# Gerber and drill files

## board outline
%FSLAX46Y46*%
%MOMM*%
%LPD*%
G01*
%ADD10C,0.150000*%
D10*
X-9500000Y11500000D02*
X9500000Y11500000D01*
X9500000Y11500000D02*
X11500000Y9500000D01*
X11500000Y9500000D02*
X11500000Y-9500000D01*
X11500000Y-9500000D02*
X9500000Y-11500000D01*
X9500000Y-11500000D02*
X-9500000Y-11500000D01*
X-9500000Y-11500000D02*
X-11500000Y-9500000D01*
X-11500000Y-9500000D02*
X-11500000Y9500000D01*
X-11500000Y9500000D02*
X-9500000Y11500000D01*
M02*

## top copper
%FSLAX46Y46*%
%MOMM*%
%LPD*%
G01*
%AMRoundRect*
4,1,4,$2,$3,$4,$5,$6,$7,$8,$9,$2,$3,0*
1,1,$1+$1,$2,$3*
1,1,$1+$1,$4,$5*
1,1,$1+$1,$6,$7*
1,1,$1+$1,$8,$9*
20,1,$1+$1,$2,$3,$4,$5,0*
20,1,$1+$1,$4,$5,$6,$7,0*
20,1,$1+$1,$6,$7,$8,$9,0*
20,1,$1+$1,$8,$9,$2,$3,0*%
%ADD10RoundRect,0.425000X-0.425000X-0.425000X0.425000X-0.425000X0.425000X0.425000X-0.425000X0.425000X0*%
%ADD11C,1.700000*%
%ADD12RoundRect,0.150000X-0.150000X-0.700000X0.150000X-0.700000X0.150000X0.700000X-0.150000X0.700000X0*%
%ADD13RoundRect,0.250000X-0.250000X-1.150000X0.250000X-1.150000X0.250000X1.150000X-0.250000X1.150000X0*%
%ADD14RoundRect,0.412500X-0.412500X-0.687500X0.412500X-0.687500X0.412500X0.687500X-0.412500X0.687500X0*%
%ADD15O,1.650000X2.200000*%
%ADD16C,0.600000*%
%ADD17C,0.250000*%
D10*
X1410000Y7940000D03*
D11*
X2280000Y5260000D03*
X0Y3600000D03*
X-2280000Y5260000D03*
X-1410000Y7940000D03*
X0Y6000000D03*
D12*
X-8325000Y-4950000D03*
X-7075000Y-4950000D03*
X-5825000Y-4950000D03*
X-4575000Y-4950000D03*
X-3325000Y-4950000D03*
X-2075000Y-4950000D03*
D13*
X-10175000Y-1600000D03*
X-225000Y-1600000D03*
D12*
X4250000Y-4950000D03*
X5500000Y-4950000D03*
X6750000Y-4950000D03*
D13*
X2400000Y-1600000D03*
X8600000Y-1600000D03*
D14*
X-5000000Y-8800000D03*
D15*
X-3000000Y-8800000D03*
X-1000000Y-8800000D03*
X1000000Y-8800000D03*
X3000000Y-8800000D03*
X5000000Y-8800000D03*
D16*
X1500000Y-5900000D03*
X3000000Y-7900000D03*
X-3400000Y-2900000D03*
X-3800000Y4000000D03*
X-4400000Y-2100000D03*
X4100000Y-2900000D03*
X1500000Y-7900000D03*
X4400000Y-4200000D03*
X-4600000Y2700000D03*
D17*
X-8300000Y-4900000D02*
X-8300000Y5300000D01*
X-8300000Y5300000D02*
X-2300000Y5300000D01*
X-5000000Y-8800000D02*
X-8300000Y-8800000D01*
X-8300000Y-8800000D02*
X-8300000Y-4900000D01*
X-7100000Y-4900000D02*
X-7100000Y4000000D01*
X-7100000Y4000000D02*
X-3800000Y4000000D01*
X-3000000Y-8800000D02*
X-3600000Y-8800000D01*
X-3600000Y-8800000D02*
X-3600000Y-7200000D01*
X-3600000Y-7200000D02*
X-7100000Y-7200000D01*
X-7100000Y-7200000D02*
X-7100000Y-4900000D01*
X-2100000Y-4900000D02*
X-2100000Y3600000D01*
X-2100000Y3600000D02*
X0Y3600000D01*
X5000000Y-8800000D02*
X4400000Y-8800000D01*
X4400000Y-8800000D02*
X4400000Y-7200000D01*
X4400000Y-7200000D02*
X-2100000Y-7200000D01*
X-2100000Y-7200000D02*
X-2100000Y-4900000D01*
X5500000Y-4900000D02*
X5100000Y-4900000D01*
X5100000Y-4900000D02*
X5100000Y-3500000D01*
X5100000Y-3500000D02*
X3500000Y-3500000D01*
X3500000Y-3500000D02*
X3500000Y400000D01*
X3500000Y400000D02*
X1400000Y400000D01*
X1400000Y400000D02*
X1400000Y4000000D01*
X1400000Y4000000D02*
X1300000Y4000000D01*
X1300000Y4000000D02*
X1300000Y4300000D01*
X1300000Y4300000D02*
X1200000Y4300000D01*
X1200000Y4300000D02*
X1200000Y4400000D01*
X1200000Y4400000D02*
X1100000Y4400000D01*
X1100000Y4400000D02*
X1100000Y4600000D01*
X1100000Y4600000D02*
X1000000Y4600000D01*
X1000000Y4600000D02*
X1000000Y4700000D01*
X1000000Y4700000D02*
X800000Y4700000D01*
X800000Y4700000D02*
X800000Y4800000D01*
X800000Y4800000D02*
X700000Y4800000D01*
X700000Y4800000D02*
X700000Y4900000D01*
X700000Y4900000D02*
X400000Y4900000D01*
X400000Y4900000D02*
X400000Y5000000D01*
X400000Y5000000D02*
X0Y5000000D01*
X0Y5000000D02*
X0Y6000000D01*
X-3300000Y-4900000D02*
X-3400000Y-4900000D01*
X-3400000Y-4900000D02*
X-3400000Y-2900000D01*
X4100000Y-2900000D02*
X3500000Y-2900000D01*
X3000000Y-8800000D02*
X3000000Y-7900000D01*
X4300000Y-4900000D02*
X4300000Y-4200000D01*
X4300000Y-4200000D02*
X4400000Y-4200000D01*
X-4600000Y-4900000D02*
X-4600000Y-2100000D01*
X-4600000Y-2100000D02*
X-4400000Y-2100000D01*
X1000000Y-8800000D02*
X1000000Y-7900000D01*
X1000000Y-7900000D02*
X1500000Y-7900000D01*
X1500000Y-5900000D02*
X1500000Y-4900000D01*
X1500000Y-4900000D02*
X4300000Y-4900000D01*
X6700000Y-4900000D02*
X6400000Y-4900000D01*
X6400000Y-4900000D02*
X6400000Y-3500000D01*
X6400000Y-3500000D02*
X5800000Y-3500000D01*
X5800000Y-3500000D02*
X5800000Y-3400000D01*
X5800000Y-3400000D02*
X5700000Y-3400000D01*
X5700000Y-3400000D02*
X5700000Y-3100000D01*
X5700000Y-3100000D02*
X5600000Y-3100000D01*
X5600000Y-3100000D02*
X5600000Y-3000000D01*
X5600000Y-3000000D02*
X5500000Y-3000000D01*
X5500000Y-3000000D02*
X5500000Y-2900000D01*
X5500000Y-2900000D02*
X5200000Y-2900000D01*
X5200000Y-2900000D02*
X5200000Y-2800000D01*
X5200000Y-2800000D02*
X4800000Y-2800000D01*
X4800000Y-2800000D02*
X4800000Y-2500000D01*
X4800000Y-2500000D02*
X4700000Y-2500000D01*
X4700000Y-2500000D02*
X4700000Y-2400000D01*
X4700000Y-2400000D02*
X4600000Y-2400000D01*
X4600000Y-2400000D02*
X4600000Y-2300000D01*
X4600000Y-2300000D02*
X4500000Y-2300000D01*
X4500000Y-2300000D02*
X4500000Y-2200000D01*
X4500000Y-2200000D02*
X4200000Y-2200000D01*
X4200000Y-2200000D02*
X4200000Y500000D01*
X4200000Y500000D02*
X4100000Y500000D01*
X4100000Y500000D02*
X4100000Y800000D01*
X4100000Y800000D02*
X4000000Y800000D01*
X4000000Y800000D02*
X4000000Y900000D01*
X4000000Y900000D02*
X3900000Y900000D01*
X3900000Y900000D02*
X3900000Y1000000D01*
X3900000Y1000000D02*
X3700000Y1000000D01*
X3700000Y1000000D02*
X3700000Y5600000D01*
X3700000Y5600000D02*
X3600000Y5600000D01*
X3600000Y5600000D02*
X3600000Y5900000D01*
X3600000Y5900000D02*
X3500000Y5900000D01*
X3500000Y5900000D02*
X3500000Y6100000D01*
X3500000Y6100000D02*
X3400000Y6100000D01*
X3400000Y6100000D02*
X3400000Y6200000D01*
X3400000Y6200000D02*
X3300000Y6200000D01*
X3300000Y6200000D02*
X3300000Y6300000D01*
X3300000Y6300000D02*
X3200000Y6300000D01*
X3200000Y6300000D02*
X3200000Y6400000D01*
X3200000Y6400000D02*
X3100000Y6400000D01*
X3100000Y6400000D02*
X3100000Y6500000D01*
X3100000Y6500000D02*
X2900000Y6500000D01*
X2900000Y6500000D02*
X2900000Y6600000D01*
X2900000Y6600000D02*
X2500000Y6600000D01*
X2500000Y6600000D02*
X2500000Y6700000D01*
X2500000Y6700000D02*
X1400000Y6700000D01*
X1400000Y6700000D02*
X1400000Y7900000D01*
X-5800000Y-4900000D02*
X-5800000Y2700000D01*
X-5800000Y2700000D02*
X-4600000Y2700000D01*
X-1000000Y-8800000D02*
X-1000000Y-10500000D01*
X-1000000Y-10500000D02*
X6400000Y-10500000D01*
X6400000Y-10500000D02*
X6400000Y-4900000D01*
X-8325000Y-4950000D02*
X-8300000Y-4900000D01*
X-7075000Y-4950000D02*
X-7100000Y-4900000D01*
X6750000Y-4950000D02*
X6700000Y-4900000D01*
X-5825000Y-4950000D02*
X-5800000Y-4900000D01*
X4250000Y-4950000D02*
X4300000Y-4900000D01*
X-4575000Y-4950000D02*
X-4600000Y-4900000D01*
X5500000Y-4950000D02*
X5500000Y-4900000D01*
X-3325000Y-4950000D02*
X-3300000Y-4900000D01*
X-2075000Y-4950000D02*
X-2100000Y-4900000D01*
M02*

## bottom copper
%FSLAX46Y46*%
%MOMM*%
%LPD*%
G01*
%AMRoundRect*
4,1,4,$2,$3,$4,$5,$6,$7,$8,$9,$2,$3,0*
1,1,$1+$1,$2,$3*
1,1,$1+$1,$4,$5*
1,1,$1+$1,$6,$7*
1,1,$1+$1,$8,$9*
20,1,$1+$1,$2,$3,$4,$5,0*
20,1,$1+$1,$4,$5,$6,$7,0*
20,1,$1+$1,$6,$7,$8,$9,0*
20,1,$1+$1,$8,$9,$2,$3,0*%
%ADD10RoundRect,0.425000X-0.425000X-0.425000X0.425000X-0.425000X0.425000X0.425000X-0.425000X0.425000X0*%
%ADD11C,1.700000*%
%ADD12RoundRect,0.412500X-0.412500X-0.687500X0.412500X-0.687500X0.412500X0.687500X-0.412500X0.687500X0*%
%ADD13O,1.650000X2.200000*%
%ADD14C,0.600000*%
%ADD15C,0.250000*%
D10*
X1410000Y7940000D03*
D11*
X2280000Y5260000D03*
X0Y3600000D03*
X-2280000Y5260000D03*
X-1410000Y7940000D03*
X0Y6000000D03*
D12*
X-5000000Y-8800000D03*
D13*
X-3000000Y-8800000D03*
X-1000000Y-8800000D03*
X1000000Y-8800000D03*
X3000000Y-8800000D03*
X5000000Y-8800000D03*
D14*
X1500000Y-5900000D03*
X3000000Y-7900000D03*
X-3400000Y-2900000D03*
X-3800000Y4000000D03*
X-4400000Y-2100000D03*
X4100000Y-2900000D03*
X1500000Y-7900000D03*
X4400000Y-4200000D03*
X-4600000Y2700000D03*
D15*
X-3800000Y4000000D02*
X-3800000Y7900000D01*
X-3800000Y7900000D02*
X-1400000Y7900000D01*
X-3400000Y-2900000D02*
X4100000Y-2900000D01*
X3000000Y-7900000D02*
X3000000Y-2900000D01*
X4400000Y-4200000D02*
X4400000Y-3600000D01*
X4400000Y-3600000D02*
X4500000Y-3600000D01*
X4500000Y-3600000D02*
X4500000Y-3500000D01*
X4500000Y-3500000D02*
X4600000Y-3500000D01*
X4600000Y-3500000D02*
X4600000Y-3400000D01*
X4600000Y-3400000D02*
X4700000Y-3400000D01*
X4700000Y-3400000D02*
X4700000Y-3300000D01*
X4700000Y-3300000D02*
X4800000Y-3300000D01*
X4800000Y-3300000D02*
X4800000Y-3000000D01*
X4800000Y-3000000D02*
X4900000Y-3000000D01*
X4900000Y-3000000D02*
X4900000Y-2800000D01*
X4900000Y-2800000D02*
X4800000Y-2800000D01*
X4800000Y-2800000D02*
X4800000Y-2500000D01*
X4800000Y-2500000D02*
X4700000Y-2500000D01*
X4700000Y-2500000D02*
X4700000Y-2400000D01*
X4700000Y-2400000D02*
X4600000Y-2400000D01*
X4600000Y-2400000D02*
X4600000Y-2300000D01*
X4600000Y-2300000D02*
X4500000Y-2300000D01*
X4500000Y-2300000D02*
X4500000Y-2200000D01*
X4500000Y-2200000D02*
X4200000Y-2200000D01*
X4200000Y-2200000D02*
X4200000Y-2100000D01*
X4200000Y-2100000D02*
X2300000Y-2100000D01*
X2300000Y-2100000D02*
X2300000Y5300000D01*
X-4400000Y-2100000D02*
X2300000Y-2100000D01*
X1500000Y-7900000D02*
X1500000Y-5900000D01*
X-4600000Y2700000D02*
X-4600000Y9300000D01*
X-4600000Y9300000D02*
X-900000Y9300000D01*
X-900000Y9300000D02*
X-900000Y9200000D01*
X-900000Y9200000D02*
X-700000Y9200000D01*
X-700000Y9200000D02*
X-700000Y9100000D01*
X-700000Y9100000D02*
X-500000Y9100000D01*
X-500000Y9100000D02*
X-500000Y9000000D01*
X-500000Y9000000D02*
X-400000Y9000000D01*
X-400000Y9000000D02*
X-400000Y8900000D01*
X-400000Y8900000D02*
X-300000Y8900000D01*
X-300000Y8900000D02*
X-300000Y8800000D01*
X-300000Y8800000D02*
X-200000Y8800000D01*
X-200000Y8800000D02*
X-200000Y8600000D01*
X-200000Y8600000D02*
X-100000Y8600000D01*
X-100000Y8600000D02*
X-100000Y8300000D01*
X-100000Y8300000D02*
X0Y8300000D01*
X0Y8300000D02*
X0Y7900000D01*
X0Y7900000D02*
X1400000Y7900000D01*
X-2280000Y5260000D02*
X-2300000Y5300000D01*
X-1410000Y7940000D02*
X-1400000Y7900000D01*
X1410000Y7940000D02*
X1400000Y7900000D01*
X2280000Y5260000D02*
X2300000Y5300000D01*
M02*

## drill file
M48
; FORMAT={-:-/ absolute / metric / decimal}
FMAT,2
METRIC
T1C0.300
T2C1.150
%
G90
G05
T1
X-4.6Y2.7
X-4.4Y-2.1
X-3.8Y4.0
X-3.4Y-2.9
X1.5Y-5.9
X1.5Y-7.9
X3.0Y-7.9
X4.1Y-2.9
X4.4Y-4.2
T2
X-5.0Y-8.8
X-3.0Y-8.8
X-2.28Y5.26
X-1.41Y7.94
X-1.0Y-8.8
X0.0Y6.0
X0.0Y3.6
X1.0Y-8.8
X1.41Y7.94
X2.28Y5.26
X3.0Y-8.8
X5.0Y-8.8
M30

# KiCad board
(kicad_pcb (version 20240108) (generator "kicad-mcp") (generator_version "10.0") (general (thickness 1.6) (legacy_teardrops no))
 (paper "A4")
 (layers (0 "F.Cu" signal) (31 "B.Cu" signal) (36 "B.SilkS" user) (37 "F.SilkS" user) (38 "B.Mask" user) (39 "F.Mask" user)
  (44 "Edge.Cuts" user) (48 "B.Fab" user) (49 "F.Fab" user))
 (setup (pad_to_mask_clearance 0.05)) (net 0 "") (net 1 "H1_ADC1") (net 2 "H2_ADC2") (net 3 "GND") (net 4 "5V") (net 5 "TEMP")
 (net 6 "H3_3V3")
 (gr_line (start -9.5 -11.5) (end 9.5 -11.5) (stroke (width 0.15) (type solid)) (layer "Edge.Cuts"))
 (gr_line (start 9.5 -11.5) (end 11.5 -9.5) (stroke (width 0.15) (type solid)) (layer "Edge.Cuts"))
 (gr_line (start 11.5 -9.5) (end 11.5 9.5) (stroke (width 0.15) (type solid)) (layer "Edge.Cuts"))
 (gr_line (start 11.5 9.5) (end 9.5 11.5) (stroke (width 0.15) (type solid)) (layer "Edge.Cuts"))
 (gr_line (start 9.5 11.5) (end -9.5 11.5) (stroke (width 0.15) (type solid)) (layer "Edge.Cuts"))
 (gr_line (start -9.5 11.5) (end -11.5 9.5) (stroke (width 0.15) (type solid)) (layer "Edge.Cuts"))
 (gr_line (start -11.5 9.5) (end -11.5 -9.5) (stroke (width 0.15) (type solid)) (layer "Edge.Cuts"))
 (gr_line (start -11.5 -9.5) (end -9.5 -11.5) (stroke (width 0.15) (type solid)) (layer "Edge.Cuts"))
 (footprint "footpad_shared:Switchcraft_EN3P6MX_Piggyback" (layer "F.Cu") (at 0 -6.0 0)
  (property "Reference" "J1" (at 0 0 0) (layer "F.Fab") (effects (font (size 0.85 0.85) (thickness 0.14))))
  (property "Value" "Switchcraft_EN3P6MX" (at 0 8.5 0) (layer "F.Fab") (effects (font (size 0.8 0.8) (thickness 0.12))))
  (pad "1" thru_hole roundrect (at 1.41 -1.94) (size 1.7 1.7) (drill 1.15) (layers "*.Cu" "*.Mask") (roundrect_rratio 0.25)
   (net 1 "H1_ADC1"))
  (pad "2" thru_hole circle (at 2.28 0.74) (size 1.7 1.7) (drill 1.15) (layers "*.Cu" "*.Mask") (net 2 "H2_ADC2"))
  (pad "3" thru_hole circle (at 0 2.4) (size 1.7 1.7) (drill 1.15) (layers "*.Cu" "*.Mask") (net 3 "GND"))
  (pad "4" thru_hole circle (at -2.28 0.74) (size 1.7 1.7) (drill 1.15) (layers "*.Cu" "*.Mask") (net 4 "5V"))
  (pad "5" thru_hole circle (at -1.41 -1.94) (size 1.7 1.7) (drill 1.15) (layers "*.Cu" "*.Mask") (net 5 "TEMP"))
  (pad "6" thru_hole circle (at 0 0) (size 1.7 1.7) (drill 1.15) (layers "*.Cu" "*.Mask") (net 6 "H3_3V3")))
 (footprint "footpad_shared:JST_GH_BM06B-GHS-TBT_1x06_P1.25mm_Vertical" (layer "F.Cu") (at -5.2 3.0 0)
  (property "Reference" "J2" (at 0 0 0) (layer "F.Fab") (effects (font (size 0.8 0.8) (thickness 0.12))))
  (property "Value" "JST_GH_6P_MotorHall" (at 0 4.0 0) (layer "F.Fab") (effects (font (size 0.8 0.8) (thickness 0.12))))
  (pad "1" smd roundrect (at -3.125 1.95) (size 0.6 1.7) (layers "F.Cu" "F.Mask" "F.Paste") (roundrect_rratio 0.25) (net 4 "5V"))
  (pad "2" smd roundrect (at -1.875 1.95) (size 0.6 1.7) (layers "F.Cu" "F.Mask" "F.Paste") (roundrect_rratio 0.25) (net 5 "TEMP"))
  (pad "3" smd roundrect (at -0.625 1.95) (size 0.6 1.7) (layers "F.Cu" "F.Mask" "F.Paste") (roundrect_rratio 0.25) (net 1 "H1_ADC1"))
  (pad "4" smd roundrect (at 0.625 1.95) (size 0.6 1.7) (layers "F.Cu" "F.Mask" "F.Paste") (roundrect_rratio 0.25) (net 2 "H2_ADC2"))
  (pad "5" smd roundrect (at 1.875 1.95) (size 0.6 1.7) (layers "F.Cu" "F.Mask" "F.Paste") (roundrect_rratio 0.25) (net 6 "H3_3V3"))
  (pad "6" smd roundrect (at 3.125 1.95) (size 0.6 1.7) (layers "F.Cu" "F.Mask" "F.Paste") (roundrect_rratio 0.25) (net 3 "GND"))
  (pad "MP" smd roundrect (at -4.975 -1.4) (size 1 2.8) (layers "F.Cu" "F.Mask" "F.Paste") (roundrect_rratio 0.25) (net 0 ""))
  (pad "MP" smd roundrect (at 4.975 -1.4) (size 1 2.8) (layers "F.Cu" "F.Mask" "F.Paste") (roundrect_rratio 0.25) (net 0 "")))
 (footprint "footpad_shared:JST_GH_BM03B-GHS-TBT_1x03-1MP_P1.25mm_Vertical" (layer "F.Cu") (at 5.5 3.0 0)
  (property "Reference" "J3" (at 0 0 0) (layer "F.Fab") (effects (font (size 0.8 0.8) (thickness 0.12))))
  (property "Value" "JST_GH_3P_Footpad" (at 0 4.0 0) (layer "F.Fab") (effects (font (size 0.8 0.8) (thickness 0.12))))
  (pad "1" smd roundrect (at -1.25 1.95) (size 0.6 1.7) (layers "F.Cu" "F.Mask" "F.Paste") (roundrect_rratio 0.25) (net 2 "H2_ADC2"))
  (pad "2" smd roundrect (at 0 1.95) (size 0.6 1.7) (layers "F.Cu" "F.Mask" "F.Paste") (roundrect_rratio 0.25) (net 6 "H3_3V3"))
  (pad "3" smd roundrect (at 1.25 1.95) (size 0.6 1.7) (layers "F.Cu" "F.Mask" "F.Paste") (roundrect_rratio 0.25) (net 1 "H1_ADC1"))
  (pad "MP" smd roundrect (at -3.1 -1.4) (size 1 2.8) (layers "F.Cu" "F.Mask" "F.Paste") (roundrect_rratio 0.25) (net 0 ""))
  (pad "MP" smd roundrect (at 3.1 -1.4) (size 1 2.8) (layers "F.Cu" "F.Mask" "F.Paste") (roundrect_rratio 0.25) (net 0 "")))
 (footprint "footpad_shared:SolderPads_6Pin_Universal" (layer "F.Cu") (at 0 8.8 0)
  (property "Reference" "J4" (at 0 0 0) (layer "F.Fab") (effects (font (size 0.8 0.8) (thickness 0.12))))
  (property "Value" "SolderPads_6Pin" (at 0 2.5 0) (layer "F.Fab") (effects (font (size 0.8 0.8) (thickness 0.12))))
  (pad "1" thru_hole roundrect (at -5 0) (size 1.65 2.2) (drill 1.15) (layers "*.Cu" "*.Mask") (roundrect_rratio 0.25) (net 4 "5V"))
  (pad "2" thru_hole oval (at -3 0) (size 1.65 2.2) (drill 1.15) (layers "*.Cu" "*.Mask") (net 5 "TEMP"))
  (pad "3" thru_hole oval (at -1 0) (size 1.65 2.2) (drill 1.15) (layers "*.Cu" "*.Mask") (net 1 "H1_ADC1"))
  (pad "4" thru_hole oval (at 1 0) (size 1.65 2.2) (drill 1.15) (layers "*.Cu" "*.Mask") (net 2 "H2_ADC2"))
  (pad "5" thru_hole oval (at 3 0) (size 1.65 2.2) (drill 1.15) (layers "*.Cu" "*.Mask") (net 6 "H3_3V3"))
  (pad "6" thru_hole oval (at 5 0) (size 1.65 2.2) (drill 1.15) (layers "*.Cu" "*.Mask") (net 3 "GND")))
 (segment (start -8.3 4.9) (end -8.3 -5.3) (width 0.25) (layer "F.Cu") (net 4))
 (segment (start -8.3 -5.3) (end -2.3 -5.3) (width 0.25) (layer "F.Cu") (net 4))
 (segment (start -5.0 8.8) (end -8.3 8.8) (width 0.25) (layer "F.Cu") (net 4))
 (segment (start -8.3 8.8) (end -8.3 4.9) (width 0.25) (layer "F.Cu") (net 4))
 (segment (start -7.1 4.9) (end -7.1 -4.0) (width 0.25) (layer "F.Cu") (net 5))
 (segment (start -7.1 -4.0) (end -3.8 -4.0) (width 0.25) (layer "F.Cu") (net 5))
 (segment (start -3.8 -4.0) (end -3.8 -7.9) (width 0.25) (layer "B.Cu") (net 5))
 (segment (start -3.8 -7.9) (end -1.4 -7.9) (width 0.25) (layer "B.Cu") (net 5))
 (segment (start -3.0 8.8) (end -3.6 8.8) (width 0.25) (layer "F.Cu") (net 5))
 (segment (start -3.6 8.8) (end -3.6 7.2) (width 0.25) (layer "F.Cu") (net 5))
 (segment (start -3.6 7.2) (end -7.1 7.2) (width 0.25) (layer "F.Cu") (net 5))
 (segment (start -7.1 7.2) (end -7.1 4.9) (width 0.25) (layer "F.Cu") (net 5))
 (segment (start -2.1 4.9) (end -2.1 -3.6) (width 0.25) (layer "F.Cu") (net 3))
 (segment (start -2.1 -3.6) (end 0.0 -3.6) (width 0.25) (layer "F.Cu") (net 3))
 (segment (start 5.0 8.8) (end 4.4 8.8) (width 0.25) (layer "F.Cu") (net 3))
 (segment (start 4.4 8.8) (end 4.4 7.2) (width 0.25) (layer "F.Cu") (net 3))
 (segment (start 4.4 7.2) (end -2.1 7.2) (width 0.25) (layer "F.Cu") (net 3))
 (segment (start -2.1 7.2) (end -2.1 4.9) (width 0.25) (layer "F.Cu") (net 3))
 (segment (start 5.5 4.9) (end 5.1 4.9) (width 0.25) (layer "F.Cu") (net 6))
 (segment (start 5.1 4.9) (end 5.1 3.5) (width 0.25) (layer "F.Cu") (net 6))
 (segment (start 5.1 3.5) (end 3.5 3.5) (width 0.25) (layer "F.Cu") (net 6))
 (segment (start 3.5 3.5) (end 3.5 -0.4) (width 0.25) (layer "F.Cu") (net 6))
 (segment (start 3.5 -0.4) (end 1.4 -0.4) (width 0.25) (layer "F.Cu") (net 6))
 (segment (start 1.4 -0.4) (end 1.4 -4.0) (width 0.25) (layer "F.Cu") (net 6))
 (segment (start 1.4 -4.0) (end 1.3 -4.0) (width 0.25) (layer "F.Cu") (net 6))
 (segment (start 1.3 -4.0) (end 1.3 -4.3) (width 0.25) (layer "F.Cu") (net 6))
 (segment (start 1.3 -4.3) (end 1.2 -4.3) (width 0.25) (layer "F.Cu") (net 6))
 (segment (start 1.2 -4.3) (end 1.2 -4.4) (width 0.25) (layer "F.Cu") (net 6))
 (segment (start 1.2 -4.4) (end 1.1 -4.4) (width 0.25) (layer "F.Cu") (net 6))
 (segment (start 1.1 -4.4) (end 1.1 -4.6) (width 0.25) (layer "F.Cu") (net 6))
 (segment (start 1.1 -4.6) (end 1.0 -4.6) (width 0.25) (layer "F.Cu") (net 6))
 (segment (start 1.0 -4.6) (end 1.0 -4.7) (width 0.25) (layer "F.Cu") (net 6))
 (segment (start 1.0 -4.7) (end 0.8 -4.7) (width 0.25) (layer "F.Cu") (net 6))
 (segment (start 0.8 -4.7) (end 0.8 -4.8) (width 0.25) (layer "F.Cu") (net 6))
 (segment (start 0.8 -4.8) (end 0.7 -4.8) (width 0.25) (layer "F.Cu") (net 6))
 (segment (start 0.7 -4.8) (end 0.7 -4.9) (width 0.25) (layer "F.Cu") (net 6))
 (segment (start 0.7 -4.9) (end 0.4 -4.9) (width 0.25) (layer "F.Cu") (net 6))
 (segment (start 0.4 -4.9) (end 0.4 -5.0) (width 0.25) (layer "F.Cu") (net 6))
 (segment (start 0.4 -5.0) (end 0.0 -5.0) (width 0.25) (layer "F.Cu") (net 6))
 (segment (start 0.0 -5.0) (end 0.0 -6.0) (width 0.25) (layer "F.Cu") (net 6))
 (segment (start -3.3 4.9) (end -3.4 4.9) (width 0.25) (layer "F.Cu") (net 6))
 (segment (start -3.4 4.9) (end -3.4 2.9) (width 0.25) (layer "F.Cu") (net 6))
 (segment (start -3.4 2.9) (end 4.1 2.9) (width 0.25) (layer "B.Cu") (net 6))
 (segment (start 4.1 2.9) (end 3.5 2.9) (width 0.25) (layer "F.Cu") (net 6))
 (segment (start 3.0 8.8) (end 3.0 7.9) (width 0.25) (layer "F.Cu") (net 6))
 (segment (start 3.0 7.9) (end 3.0 2.9) (width 0.25) (layer "B.Cu") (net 6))
 (segment (start 4.3 4.9) (end 4.3 4.2) (width 0.25) (layer "F.Cu") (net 2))
 (segment (start 4.3 4.2) (end 4.4 4.2) (width 0.25) (layer "F.Cu") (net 2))
 (segment (start 4.4 4.2) (end 4.4 3.6) (width 0.25) (layer "B.Cu") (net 2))
 (segment (start 4.4 3.6) (end 4.5 3.6) (width 0.25) (layer "B.Cu") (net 2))
 (segment (start 4.5 3.6) (end 4.5 3.5) (width 0.25) (layer "B.Cu") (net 2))
 (segment (start 4.5 3.5) (end 4.6 3.5) (width 0.25) (layer "B.Cu") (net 2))
 (segment (start 4.6 3.5) (end 4.6 3.4) (width 0.25) (layer "B.Cu") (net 2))
 (segment (start 4.6 3.4) (end 4.7 3.4) (width 0.25) (layer "B.Cu") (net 2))
 (segment (start 4.7 3.4) (end 4.7 3.3) (width 0.25) (layer "B.Cu") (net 2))
 (segment (start 4.7 3.3) (end 4.8 3.3) (width 0.25) (layer "B.Cu") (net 2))
 (segment (start 4.8 3.3) (end 4.8 3.0) (width 0.25) (layer "B.Cu") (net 2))
 (segment (start 4.8 3.0) (end 4.9 3.0) (width 0.25) (layer "B.Cu") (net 2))
 (segment (start 4.9 3.0) (end 4.9 2.8) (width 0.25) (layer "B.Cu") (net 2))
 (segment (start 4.9 2.8) (end 4.8 2.8) (width 0.25) (layer "B.Cu") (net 2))
 (segment (start 4.8 2.8) (end 4.8 2.5) (width 0.25) (layer "B.Cu") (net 2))
 (segment (start 4.8 2.5) (end 4.7 2.5) (width 0.25) (layer "B.Cu") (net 2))
 (segment (start 4.7 2.5) (end 4.7 2.4) (width 0.25) (layer "B.Cu") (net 2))
 (segment (start 4.7 2.4) (end 4.6 2.4) (width 0.25) (layer "B.Cu") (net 2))
 (segment (start 4.6 2.4) (end 4.6 2.3) (width 0.25) (layer "B.Cu") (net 2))
 (segment (start 4.6 2.3) (end 4.5 2.3) (width 0.25) (layer "B.Cu") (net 2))
 (segment (start 4.5 2.3) (end 4.5 2.2) (width 0.25) (layer "B.Cu") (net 2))
 (segment (start 4.5 2.2) (end 4.2 2.2) (width 0.25) (layer "B.Cu") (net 2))
 (segment (start 4.2 2.2) (end 4.2 2.1) (width 0.25) (layer "B.Cu") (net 2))
 (segment (start 4.2 2.1) (end 2.3 2.1) (width 0.25) (layer "B.Cu") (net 2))
 (segment (start 2.3 2.1) (end 2.3 -5.3) (width 0.25) (layer "B.Cu") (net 2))
 (segment (start -4.6 4.9) (end -4.6 2.1) (width 0.25) (layer "F.Cu") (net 2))
 (segment (start -4.6 2.1) (end -4.4 2.1) (width 0.25) (layer "F.Cu") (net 2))
 (segment (start -4.4 2.1) (end 2.3 2.1) (width 0.25) (layer "B.Cu") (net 2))
 (segment (start 1.0 8.8) (end 1.0 7.9) (width 0.25) (layer "F.Cu") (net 2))
 (segment (start 1.0 7.9) (end 1.5 7.9) (width 0.25) (layer "F.Cu") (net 2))
 (segment (start 1.5 7.9) (end 1.5 5.9) (width 0.25) (layer "B.Cu") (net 2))
 (segment (start 1.5 5.9) (end 1.5 4.9) (width 0.25) (layer "F.Cu") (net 2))
 (segment (start 1.5 4.9) (end 4.3 4.9) (width 0.25) (layer "F.Cu") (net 2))
 (segment (start 6.7 4.9) (end 6.4 4.9) (width 0.25) (layer "F.Cu") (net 1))
 (segment (start 6.4 4.9) (end 6.4 3.5) (width 0.25) (layer "F.Cu") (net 1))
 (segment (start 6.4 3.5) (end 5.8 3.5) (width 0.25) (layer "F.Cu") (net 1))
 (segment (start 5.8 3.5) (end 5.8 3.4) (width 0.25) (layer "F.Cu") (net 1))
 (segment (start 5.8 3.4) (end 5.7 3.4) (width 0.25) (layer "F.Cu") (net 1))
 (segment (start 5.7 3.4) (end 5.7 3.1) (width 0.25) (layer "F.Cu") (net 1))
 (segment (start 5.7 3.1) (end 5.6 3.1) (width 0.25) (layer "F.Cu") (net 1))
 (segment (start 5.6 3.1) (end 5.6 3.0) (width 0.25) (layer "F.Cu") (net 1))
 (segment (start 5.6 3.0) (end 5.5 3.0) (width 0.25) (layer "F.Cu") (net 1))
 (segment (start 5.5 3.0) (end 5.5 2.9) (width 0.25) (layer "F.Cu") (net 1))
 (segment (start 5.5 2.9) (end 5.2 2.9) (width 0.25) (layer "F.Cu") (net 1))
 (segment (start 5.2 2.9) (end 5.2 2.8) (width 0.25) (layer "F.Cu") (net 1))
 (segment (start 5.2 2.8) (end 4.8 2.8) (width 0.25) (layer "F.Cu") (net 1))
 (segment (start 4.8 2.8) (end 4.8 2.5) (width 0.25) (layer "F.Cu") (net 1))
 (segment (start 4.8 2.5) (end 4.7 2.5) (width 0.25) (layer "F.Cu") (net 1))
 (segment (start 4.7 2.5) (end 4.7 2.4) (width 0.25) (layer "F.Cu") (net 1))
 (segment (start 4.7 2.4) (end 4.6 2.4) (width 0.25) (layer "F.Cu") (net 1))
 (segment (start 4.6 2.4) (end 4.6 2.3) (width 0.25) (layer "F.Cu") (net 1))
 (segment (start 4.6 2.3) (end 4.5 2.3) (width 0.25) (layer "F.Cu") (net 1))
 (segment (start 4.5 2.3) (end 4.5 2.2) (width 0.25) (layer "F.Cu") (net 1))
 (segment (start 4.5 2.2) (end 4.2 2.2) (width 0.25) (layer "F.Cu") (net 1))
 (segment (start 4.2 2.2) (end 4.2 -0.5) (width 0.25) (layer "F.Cu") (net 1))
 (segment (start 4.2 -0.5) (end 4.1 -0.5) (width 0.25) (layer "F.Cu") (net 1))
 (segment (start 4.1 -0.5) (end 4.1 -0.8) (width 0.25) (layer "F.Cu") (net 1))
 (segment (start 4.1 -0.8) (end 4.0 -0.8) (width 0.25) (layer "F.Cu") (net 1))
 (segment (start 4.0 -0.8) (end 4.0 -0.9) (width 0.25) (layer "F.Cu") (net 1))
 (segment (start 4.0 -0.9) (end 3.9 -0.9) (width 0.25) (layer "F.Cu") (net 1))
 (segment (start 3.9 -0.9) (end 3.9 -1.0) (width 0.25) (layer "F.Cu") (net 1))
 (segment (start 3.9 -1.0) (end 3.7 -1.0) (width 0.25) (layer "F.Cu") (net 1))
 (segment (start 3.7 -1.0) (end 3.7 -5.6) (width 0.25) (layer "F.Cu") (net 1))
 (segment (start 3.7 -5.6) (end 3.6 -5.6) (width 0.25) (layer "F.Cu") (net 1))
 (segment (start 3.6 -5.6) (end 3.6 -5.9) (width 0.25) (layer "F.Cu") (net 1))
 (segment (start 3.6 -5.9) (end 3.5 -5.9) (width 0.25) (layer "F.Cu") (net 1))
 (segment (start 3.5 -5.9) (end 3.5 -6.1) (width 0.25) (layer "F.Cu") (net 1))
 (segment (start 3.5 -6.1) (end 3.4 -6.1) (width 0.25) (layer "F.Cu") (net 1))
 (segment (start 3.4 -6.1) (end 3.4 -6.2) (width 0.25) (layer "F.Cu") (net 1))
 (segment (start 3.4 -6.2) (end 3.3 -6.2) (width 0.25) (layer "F.Cu") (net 1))
 (segment (start 3.3 -6.2) (end 3.3 -6.3) (width 0.25) (layer "F.Cu") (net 1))
 (segment (start 3.3 -6.3) (end 3.2 -6.3) (width 0.25) (layer "F.Cu") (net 1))
 (segment (start 3.2 -6.3) (end 3.2 -6.4) (width 0.25) (layer "F.Cu") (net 1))
 (segment (start 3.2 -6.4) (end 3.1 -6.4) (width 0.25) (layer "F.Cu") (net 1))
 (segment (start 3.1 -6.4) (end 3.1 -6.5) (width 0.25) (layer "F.Cu") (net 1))
 (segment (start 3.1 -6.5) (end 2.9 -6.5) (width 0.25) (layer "F.Cu") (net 1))
 (segment (start 2.9 -6.5) (end 2.9 -6.6) (width 0.25) (layer "F.Cu") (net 1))
 (segment (start 2.9 -6.6) (end 2.5 -6.6) (width 0.25) (layer "F.Cu") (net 1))
 (segment (start 2.5 -6.6) (end 2.5 -6.7) (width 0.25) (layer "F.Cu") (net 1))
 (segment (start 2.5 -6.7) (end 1.4 -6.7) (width 0.25) (layer "F.Cu") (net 1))
 (segment (start 1.4 -6.7) (end 1.4 -7.9) (width 0.25) (layer "F.Cu") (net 1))
 (segment (start -5.8 4.9) (end -5.8 -2.7) (width 0.25) (layer "F.Cu") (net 1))
 (segment (start -5.8 -2.7) (end -4.6 -2.7) (width 0.25) (layer "F.Cu") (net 1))
 (segment (start -4.6 -2.7) (end -4.6 -9.3) (width 0.25) (layer "B.Cu") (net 1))
 (segment (start -4.6 -9.3) (end -0.9 -9.3) (width 0.25) (layer "B.Cu") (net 1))
 (segment (start -0.9 -9.3) (end -0.9 -9.2) (width 0.25) (layer "B.Cu") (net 1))
 (segment (start -0.9 -9.2) (end -0.7 -9.2) (width 0.25) (layer "B.Cu") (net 1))
 (segment (start -0.7 -9.2) (end -0.7 -9.1) (width 0.25) (layer "B.Cu") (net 1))
 (segment (start -0.7 -9.1) (end -0.5 -9.1) (width 0.25) (layer "B.Cu") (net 1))
 (segment (start -0.5 -9.1) (end -0.5 -9.0) (width 0.25) (layer "B.Cu") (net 1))
 (segment (start -0.5 -9.0) (end -0.4 -9.0) (width 0.25) (layer "B.Cu") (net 1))
 (segment (start -0.4 -9.0) (end -0.4 -8.9) (width 0.25) (layer "B.Cu") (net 1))
 (segment (start -0.4 -8.9) (end -0.3 -8.9) (width 0.25) (layer "B.Cu") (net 1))
 (segment (start -0.3 -8.9) (end -0.3 -8.8) (width 0.25) (layer "B.Cu") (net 1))
 (segment (start -0.3 -8.8) (end -0.2 -8.8) (width 0.25) (layer "B.Cu") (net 1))
 (segment (start -0.2 -8.8) (end -0.2 -8.6) (width 0.25) (layer "B.Cu") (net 1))
 (segment (start -0.2 -8.6) (end -0.1 -8.6) (width 0.25) (layer "B.Cu") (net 1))
 (segment (start -0.1 -8.6) (end -0.1 -8.3) (width 0.25) (layer "B.Cu") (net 1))
 (segment (start -0.1 -8.3) (end 0.0 -8.3) (width 0.25) (layer "B.Cu") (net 1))
 (segment (start 0.0 -8.3) (end 0.0 -7.9) (width 0.25) (layer "B.Cu") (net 1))
 (segment (start 0.0 -7.9) (end 1.4 -7.9) (width 0.25) (layer "B.Cu") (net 1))
 (segment (start -1.0 8.8) (end -1.0 10.5) (width 0.25) (layer "F.Cu") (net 1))
 (segment (start -1.0 10.5) (end 6.4 10.5) (width 0.25) (layer "F.Cu") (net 1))
 (segment (start 6.4 10.5) (end 6.4 4.9) (width 0.25) (layer "F.Cu") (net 1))
 (segment (start -2.28 -5.26) (end -2.3 -5.3) (width 0.25) (layer "B.Cu") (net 4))
 (segment (start -8.325 4.95) (end -8.3 4.9) (width 0.25) (layer "F.Cu") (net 4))
 (segment (start -1.41 -7.94) (end -1.4 -7.9) (width 0.25) (layer "B.Cu") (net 5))
 (segment (start -7.075 4.95) (end -7.1 4.9) (width 0.25) (layer "F.Cu") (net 5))
 (segment (start 1.41 -7.94) (end 1.4 -7.9) (width 0.25) (layer "B.Cu") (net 1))
 (segment (start 6.75 4.95) (end 6.7 4.9) (width 0.25) (layer "F.Cu") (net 1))
 (segment (start -5.825 4.95) (end -5.8 4.9) (width 0.25) (layer "F.Cu") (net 1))
 (segment (start 2.28 -5.26) (end 2.3 -5.3) (width 0.25) (layer "B.Cu") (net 2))
 (segment (start 4.25 4.95) (end 4.3 4.9) (width 0.25) (layer "F.Cu") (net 2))
 (segment (start -4.575 4.95) (end -4.6 4.9) (width 0.25) (layer "F.Cu") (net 2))
 (segment (start 5.5 4.95) (end 5.5 4.9) (width 0.25) (layer "F.Cu") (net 6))
 (segment (start -3.325 4.95) (end -3.3 4.9) (width 0.25) (layer "F.Cu") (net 6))
 (segment (start -2.075 4.95) (end -2.1 4.9) (width 0.25) (layer "F.Cu") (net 3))
 (via (at 1.5 5.9) (size 0.6) (drill 0.3) (layers "F.Cu" "B.Cu") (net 2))
 (via (at 3.0 7.9) (size 0.6) (drill 0.3) (layers "F.Cu" "B.Cu") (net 6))
 (via (at -3.4 2.9) (size 0.6) (drill 0.3) (layers "F.Cu" "B.Cu") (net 6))
 (via (at -3.8 -4.0) (size 0.6) (drill 0.3) (layers "F.Cu" "B.Cu") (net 5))
 (via (at -4.4 2.1) (size 0.6) (drill 0.3) (layers "F.Cu" "B.Cu") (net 2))
 (via (at 4.1 2.9) (size 0.6) (drill 0.3) (layers "F.Cu" "B.Cu") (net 6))
 (via (at 1.5 7.9) (size 0.6) (drill 0.3) (layers "F.Cu" "B.Cu") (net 2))
 (via (at 4.4 4.2) (size 0.6) (drill 0.3) (layers "F.Cu" "B.Cu") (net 2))
 (via (at -4.6 -2.7) (size 0.6) (drill 0.3) (layers "F.Cu" "B.Cu") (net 1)))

